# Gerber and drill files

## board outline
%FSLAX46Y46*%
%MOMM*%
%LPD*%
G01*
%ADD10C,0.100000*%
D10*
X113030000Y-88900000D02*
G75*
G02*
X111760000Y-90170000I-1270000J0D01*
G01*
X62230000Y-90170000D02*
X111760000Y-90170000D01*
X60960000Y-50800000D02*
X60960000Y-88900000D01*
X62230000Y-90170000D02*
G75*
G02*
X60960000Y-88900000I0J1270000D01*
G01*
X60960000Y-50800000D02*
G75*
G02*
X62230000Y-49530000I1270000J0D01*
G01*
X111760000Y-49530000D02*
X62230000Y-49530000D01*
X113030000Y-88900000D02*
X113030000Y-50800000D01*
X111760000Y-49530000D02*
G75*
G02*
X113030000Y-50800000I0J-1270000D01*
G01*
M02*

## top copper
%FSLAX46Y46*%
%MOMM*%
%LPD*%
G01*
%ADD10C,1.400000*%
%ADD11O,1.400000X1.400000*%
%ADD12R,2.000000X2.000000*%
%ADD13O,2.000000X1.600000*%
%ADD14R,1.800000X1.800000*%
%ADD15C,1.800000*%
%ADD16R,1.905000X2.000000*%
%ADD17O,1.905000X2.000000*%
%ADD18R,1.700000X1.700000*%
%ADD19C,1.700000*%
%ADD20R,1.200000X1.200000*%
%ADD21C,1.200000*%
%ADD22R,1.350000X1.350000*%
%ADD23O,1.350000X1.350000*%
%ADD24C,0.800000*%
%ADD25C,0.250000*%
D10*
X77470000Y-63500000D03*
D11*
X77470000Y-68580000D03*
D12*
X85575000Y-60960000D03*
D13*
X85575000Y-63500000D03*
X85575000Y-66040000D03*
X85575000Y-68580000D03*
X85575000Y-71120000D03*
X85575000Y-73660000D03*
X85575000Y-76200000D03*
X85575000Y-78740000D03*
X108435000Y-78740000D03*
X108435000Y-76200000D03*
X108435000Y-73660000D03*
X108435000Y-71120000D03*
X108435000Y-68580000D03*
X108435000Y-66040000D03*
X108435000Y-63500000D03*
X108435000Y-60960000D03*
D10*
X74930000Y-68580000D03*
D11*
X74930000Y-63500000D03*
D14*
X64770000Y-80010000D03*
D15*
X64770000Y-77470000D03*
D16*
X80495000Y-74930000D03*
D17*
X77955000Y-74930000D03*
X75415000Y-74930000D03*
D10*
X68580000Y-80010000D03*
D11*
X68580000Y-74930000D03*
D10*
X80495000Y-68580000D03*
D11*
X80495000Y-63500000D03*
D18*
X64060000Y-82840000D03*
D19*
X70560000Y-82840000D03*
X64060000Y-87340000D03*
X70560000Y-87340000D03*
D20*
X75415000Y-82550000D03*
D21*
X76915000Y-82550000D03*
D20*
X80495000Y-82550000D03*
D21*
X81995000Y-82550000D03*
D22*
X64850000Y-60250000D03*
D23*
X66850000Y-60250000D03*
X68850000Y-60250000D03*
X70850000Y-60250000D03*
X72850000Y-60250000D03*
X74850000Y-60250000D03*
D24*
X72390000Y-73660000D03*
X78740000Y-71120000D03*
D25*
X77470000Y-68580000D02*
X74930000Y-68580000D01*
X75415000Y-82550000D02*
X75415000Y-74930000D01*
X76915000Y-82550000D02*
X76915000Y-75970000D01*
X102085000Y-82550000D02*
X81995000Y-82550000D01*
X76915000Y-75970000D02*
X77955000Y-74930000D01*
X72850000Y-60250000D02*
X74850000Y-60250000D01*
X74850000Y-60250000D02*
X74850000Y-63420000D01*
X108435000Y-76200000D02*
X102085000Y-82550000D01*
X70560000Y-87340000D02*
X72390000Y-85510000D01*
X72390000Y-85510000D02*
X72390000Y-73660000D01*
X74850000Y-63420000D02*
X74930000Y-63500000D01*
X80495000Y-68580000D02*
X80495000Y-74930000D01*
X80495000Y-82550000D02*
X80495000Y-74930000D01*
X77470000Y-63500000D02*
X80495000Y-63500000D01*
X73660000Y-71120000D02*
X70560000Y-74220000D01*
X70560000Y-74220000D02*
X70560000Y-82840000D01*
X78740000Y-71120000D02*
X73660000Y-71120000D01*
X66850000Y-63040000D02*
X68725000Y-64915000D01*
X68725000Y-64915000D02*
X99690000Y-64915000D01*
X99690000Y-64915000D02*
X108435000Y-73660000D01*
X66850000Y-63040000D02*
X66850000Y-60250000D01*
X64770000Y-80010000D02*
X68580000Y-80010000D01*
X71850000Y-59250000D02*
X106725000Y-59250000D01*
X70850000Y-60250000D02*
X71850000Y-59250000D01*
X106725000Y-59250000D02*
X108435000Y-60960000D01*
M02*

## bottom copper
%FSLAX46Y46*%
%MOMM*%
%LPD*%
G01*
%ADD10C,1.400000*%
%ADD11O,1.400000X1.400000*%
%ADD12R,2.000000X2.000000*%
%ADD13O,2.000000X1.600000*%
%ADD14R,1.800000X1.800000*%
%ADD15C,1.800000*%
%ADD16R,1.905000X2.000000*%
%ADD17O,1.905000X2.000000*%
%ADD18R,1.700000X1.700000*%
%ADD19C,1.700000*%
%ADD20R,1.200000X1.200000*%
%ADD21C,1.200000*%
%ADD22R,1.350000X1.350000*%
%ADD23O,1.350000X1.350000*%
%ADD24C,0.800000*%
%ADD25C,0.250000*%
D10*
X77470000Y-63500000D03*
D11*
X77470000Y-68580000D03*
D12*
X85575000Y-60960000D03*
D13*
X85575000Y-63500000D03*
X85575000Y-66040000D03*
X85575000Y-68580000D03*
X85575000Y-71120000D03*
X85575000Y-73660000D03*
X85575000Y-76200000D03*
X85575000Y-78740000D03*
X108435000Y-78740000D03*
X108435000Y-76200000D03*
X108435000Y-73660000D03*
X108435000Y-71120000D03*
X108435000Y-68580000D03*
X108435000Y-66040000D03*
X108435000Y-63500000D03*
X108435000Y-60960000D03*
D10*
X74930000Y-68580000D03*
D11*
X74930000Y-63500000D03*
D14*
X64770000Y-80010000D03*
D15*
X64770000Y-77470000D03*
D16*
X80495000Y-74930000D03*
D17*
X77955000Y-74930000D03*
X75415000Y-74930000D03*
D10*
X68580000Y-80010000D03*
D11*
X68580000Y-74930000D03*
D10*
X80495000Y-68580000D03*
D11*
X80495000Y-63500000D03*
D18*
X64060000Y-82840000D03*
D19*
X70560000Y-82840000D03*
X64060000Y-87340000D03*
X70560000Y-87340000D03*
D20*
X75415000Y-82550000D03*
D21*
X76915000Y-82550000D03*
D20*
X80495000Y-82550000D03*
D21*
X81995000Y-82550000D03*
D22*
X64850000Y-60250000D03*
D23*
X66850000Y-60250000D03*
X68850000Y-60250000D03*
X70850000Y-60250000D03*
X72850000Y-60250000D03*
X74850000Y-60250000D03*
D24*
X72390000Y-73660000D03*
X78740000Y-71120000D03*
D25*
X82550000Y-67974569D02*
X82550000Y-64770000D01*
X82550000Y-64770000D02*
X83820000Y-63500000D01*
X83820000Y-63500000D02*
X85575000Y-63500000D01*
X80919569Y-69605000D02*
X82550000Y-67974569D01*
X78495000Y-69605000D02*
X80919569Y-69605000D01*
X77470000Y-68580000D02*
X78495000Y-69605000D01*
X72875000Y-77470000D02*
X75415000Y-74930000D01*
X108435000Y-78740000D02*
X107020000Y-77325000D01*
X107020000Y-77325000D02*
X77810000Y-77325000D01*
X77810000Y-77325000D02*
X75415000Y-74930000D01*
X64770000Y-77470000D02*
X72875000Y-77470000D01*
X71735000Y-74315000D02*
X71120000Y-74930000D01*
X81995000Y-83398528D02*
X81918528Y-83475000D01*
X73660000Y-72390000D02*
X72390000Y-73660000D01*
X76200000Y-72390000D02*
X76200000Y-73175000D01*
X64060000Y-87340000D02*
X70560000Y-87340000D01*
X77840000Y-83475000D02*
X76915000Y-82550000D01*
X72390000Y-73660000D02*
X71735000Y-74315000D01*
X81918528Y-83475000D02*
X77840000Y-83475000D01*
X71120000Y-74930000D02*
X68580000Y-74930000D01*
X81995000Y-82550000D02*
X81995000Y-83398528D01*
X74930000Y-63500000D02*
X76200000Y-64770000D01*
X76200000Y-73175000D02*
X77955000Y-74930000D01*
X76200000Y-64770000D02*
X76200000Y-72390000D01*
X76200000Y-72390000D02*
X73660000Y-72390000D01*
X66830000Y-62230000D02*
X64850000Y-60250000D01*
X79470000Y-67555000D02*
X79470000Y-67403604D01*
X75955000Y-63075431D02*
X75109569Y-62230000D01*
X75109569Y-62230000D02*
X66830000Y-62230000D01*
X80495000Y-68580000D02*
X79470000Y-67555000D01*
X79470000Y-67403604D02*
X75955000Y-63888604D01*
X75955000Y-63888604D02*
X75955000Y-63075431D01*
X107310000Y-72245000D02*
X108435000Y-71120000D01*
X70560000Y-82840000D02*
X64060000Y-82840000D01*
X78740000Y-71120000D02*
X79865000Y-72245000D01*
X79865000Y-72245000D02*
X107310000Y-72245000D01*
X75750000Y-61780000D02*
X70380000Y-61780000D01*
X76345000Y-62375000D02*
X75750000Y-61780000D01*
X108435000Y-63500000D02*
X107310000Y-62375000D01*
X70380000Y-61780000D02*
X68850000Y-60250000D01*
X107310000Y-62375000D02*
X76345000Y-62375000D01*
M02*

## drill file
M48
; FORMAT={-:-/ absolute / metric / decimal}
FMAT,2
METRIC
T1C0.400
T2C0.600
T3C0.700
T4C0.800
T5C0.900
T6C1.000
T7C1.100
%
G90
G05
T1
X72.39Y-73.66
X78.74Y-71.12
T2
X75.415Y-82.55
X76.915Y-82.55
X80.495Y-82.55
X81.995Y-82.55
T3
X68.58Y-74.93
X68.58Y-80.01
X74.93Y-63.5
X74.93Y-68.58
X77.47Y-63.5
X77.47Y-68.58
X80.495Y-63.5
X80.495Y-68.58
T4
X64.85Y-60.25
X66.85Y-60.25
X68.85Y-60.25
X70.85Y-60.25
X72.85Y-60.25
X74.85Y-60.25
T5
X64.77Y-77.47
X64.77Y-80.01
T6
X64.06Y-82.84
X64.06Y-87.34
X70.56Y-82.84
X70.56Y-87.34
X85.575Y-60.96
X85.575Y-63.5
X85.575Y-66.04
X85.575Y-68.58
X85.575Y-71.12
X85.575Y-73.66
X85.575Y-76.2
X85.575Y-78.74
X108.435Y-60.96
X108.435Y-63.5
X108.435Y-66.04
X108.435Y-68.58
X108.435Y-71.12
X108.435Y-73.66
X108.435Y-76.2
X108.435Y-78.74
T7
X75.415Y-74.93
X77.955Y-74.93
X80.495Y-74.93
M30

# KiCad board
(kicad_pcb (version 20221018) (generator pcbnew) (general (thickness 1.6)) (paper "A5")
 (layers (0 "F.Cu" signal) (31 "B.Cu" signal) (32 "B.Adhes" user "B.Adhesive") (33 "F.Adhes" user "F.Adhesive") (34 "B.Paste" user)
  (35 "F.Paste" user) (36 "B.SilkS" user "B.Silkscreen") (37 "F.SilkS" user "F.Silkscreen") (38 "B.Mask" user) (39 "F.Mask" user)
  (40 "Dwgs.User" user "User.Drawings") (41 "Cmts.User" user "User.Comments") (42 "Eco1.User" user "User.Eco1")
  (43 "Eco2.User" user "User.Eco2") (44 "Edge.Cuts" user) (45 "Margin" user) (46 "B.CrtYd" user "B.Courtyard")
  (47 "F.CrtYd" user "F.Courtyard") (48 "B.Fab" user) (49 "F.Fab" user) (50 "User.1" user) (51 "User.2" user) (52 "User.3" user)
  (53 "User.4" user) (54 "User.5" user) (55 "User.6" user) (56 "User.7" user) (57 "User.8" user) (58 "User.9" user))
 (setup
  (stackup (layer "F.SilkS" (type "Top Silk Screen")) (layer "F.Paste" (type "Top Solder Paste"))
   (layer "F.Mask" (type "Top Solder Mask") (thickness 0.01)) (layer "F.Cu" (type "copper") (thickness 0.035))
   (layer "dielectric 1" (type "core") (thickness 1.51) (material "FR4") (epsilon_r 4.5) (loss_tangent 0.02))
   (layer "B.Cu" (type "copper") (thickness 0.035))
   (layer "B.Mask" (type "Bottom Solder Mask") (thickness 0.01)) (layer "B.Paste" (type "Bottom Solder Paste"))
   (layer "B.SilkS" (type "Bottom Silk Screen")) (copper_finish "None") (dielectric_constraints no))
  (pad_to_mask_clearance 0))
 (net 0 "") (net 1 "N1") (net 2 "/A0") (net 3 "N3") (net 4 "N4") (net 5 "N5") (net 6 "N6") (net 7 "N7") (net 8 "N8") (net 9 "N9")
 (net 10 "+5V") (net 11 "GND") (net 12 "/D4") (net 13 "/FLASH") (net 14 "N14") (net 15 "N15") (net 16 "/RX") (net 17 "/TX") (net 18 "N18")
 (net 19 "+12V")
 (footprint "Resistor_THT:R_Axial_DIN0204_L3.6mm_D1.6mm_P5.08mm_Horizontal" (layer "F.Cu") (at 77.47 63.5 -90)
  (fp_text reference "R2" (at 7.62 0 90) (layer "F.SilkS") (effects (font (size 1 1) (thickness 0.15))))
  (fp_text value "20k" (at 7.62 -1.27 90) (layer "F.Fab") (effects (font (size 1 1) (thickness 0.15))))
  (pad "1" thru_hole circle (at 0 0 270) (size 1.4 1.4) (drill 0.7) (layers "*.Cu" "*.Mask") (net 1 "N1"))
  (pad "2" thru_hole oval (at 5.08 0 270) (size 1.4 1.4) (drill 0.7) (layers "*.Cu" "*.Mask") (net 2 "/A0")))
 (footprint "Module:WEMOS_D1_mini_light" (layer "F.Cu") (at 85.575 60.96)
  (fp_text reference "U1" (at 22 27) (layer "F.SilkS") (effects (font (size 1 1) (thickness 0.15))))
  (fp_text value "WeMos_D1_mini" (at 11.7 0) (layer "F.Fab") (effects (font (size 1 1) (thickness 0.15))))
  (pad "1" thru_hole rect (at 0 0) (size 2 2) (drill 1) (layers "*.Cu" "*.Mask") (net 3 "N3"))
  (pad "2" thru_hole oval (at 0 2.54) (size 2 1.6) (drill 1) (layers "*.Cu" "*.Mask") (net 2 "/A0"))
  (pad "3" thru_hole oval (at 0 5.08) (size 2 1.6) (drill 1) (layers "*.Cu" "*.Mask") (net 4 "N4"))
  (pad "4" thru_hole oval (at 0 7.62) (size 2 1.6) (drill 1) (layers "*.Cu" "*.Mask") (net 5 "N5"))
  (pad "5" thru_hole oval (at 0 10.16) (size 2 1.6) (drill 1) (layers "*.Cu" "*.Mask") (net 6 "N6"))
  (pad "6" thru_hole oval (at 0 12.7) (size 2 1.6) (drill 1) (layers "*.Cu" "*.Mask") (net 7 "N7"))
  (pad "7" thru_hole oval (at 0 15.24) (size 2 1.6) (drill 1) (layers "*.Cu" "*.Mask") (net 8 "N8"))
  (pad "8" thru_hole oval (at 0 17.78) (size 2 1.6) (drill 1) (layers "*.Cu" "*.Mask") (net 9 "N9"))
  (pad "9" thru_hole oval (at 22.86 17.78) (size 2 1.6) (drill 1) (layers "*.Cu" "*.Mask") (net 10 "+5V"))
  (pad "10" thru_hole oval (at 22.86 15.24) (size 2 1.6) (drill 1) (layers "*.Cu" "*.Mask") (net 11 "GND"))
  (pad "11" thru_hole oval (at 22.86 12.7) (size 2 1.6) (drill 1) (layers "*.Cu" "*.Mask") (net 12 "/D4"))
  (pad "12" thru_hole oval (at 22.86 10.16) (size 2 1.6) (drill 1) (layers "*.Cu" "*.Mask") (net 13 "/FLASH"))
  (pad "13" thru_hole oval (at 22.86 7.62) (size 2 1.6) (drill 1) (layers "*.Cu" "*.Mask") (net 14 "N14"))
  (pad "14" thru_hole oval (at 22.86 5.08) (size 2 1.6) (drill 1) (layers "*.Cu" "*.Mask") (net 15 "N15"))
  (pad "15" thru_hole oval (at 22.86 2.54) (size 2 1.6) (drill 1) (layers "*.Cu" "*.Mask") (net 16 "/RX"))
  (pad "16" thru_hole oval (at 22.86 0) (size 2 1.6) (drill 1) (layers "*.Cu" "*.Mask") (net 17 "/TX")))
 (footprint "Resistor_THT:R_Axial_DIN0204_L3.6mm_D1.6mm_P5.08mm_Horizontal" (layer "F.Cu") (at 74.93 68.58 90)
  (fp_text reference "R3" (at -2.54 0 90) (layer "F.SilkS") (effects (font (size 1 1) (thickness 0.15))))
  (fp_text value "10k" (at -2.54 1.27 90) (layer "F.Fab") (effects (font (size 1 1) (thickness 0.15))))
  (pad "1" thru_hole circle (at 0 0 90) (size 1.4 1.4) (drill 0.7) (layers "*.Cu" "*.Mask") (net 2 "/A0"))
  (pad "2" thru_hole oval (at 5.08 0 90) (size 1.4 1.4) (drill 0.7) (layers "*.Cu" "*.Mask") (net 11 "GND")))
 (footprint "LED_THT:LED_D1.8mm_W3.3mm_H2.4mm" (layer "F.Cu") (at 64.77 80.01 90)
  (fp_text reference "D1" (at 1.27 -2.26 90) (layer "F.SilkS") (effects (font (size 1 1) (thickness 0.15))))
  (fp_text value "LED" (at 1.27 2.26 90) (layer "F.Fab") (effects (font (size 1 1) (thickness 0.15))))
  (pad "1" thru_hole rect (at 0 0 90) (size 1.8 1.8) (drill 0.9) (layers "*.Cu" "*.Mask") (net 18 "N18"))
  (pad "2" thru_hole circle (at 2.54 0 90) (size 1.8 1.8) (drill 0.9) (layers "*.Cu" "*.Mask") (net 10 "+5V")))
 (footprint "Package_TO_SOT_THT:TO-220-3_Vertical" (layer "F.Cu") (at 80.495 74.93 180)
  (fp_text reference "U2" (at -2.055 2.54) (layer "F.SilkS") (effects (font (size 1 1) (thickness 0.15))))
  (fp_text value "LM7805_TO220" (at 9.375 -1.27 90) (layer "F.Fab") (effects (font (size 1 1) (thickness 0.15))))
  (pad "1" thru_hole rect (at 0 0 180) (size 1.905 2) (drill 1.1) (layers "*.Cu" "*.Mask") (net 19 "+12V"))
  (pad "2" thru_hole oval (at 2.54 0 180) (size 1.905 2) (drill 1.1) (layers "*.Cu" "*.Mask") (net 11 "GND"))
  (pad "3" thru_hole oval (at 5.08 0 180) (size 1.905 2) (drill 1.1) (layers "*.Cu" "*.Mask") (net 10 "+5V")))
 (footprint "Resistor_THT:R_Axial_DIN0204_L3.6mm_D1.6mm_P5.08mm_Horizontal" (layer "F.Cu") (at 68.58 80.01 90)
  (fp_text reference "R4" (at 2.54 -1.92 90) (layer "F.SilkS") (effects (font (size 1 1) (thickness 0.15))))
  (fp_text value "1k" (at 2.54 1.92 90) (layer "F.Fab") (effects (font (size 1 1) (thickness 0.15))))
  (pad "1" thru_hole circle (at 0 0 90) (size 1.4 1.4) (drill 0.7) (layers "*.Cu" "*.Mask") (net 18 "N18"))
  (pad "2" thru_hole oval (at 5.08 0 90) (size 1.4 1.4) (drill 0.7) (layers "*.Cu" "*.Mask") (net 11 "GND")))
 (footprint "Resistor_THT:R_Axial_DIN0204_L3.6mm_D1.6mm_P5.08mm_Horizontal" (layer "F.Cu") (at 80.495 68.58 90)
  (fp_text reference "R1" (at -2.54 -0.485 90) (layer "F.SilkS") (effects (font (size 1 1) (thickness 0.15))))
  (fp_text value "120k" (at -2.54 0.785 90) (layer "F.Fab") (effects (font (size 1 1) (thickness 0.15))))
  (pad "1" thru_hole circle (at 0 0 90) (size 1.4 1.4) (drill 0.7) (layers "*.Cu" "*.Mask") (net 19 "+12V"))
  (pad "2" thru_hole oval (at 5.08 0 90) (size 1.4 1.4) (drill 0.7) (layers "*.Cu" "*.Mask") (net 1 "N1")))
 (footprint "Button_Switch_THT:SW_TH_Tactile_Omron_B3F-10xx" (layer "F.Cu") (at 64.06 82.84)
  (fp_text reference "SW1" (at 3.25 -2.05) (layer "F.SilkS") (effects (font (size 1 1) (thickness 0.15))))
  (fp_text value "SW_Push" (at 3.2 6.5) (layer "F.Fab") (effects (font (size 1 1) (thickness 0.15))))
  (pad "1" thru_hole rect (at 0 0) (size 1.7 1.7) (drill 1) (layers "*.Cu" "*.Mask") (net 13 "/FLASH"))
  (pad "1" thru_hole circle (at 6.5 0) (size 1.7 1.7) (drill 1) (layers "*.Cu" "*.Mask") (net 13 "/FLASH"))
  (pad "2" thru_hole circle (at 0 4.5) (size 1.7 1.7) (drill 1) (layers "*.Cu" "*.Mask") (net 11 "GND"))
  (pad "2" thru_hole circle (at 6.5 4.5) (size 1.7 1.7) (drill 1) (layers "*.Cu" "*.Mask") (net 11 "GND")))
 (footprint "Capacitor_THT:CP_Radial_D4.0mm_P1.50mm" (layer "F.Cu") (at 75.415 82.55)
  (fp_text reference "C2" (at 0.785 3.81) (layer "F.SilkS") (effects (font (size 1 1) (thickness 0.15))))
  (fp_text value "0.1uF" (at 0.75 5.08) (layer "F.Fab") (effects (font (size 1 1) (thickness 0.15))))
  (pad "1" thru_hole rect (at 0 0) (size 1.2 1.2) (drill 0.6) (layers "*.Cu" "*.Mask") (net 10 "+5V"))
  (pad "2" thru_hole circle (at 1.5 0) (size 1.2 1.2) (drill 0.6) (layers "*.Cu" "*.Mask") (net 11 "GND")))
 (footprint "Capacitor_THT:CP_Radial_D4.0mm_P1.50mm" (layer "F.Cu") (at 80.495 82.55)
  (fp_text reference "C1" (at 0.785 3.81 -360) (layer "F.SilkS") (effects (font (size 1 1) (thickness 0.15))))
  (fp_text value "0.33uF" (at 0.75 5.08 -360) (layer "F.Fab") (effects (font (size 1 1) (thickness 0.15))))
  (pad "1" thru_hole rect (at 0 0) (size 1.2 1.2) (drill 0.6) (layers "*.Cu" "*.Mask") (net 19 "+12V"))
  (pad "2" thru_hole circle (at 1.5 0) (size 1.2 1.2) (drill 0.6) (layers "*.Cu" "*.Mask") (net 11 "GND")))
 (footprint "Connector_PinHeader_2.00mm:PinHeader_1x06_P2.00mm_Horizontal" (layer "F.Cu") (at 64.85 60.25 90)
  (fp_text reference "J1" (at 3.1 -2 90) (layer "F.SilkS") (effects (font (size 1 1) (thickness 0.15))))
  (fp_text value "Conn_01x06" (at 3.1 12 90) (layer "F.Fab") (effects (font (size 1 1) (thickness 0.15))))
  (pad "1" thru_hole rect (at 0 0 90) (size 1.35 1.35) (drill 0.8) (layers "*.Cu" "*.Mask") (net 19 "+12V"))
  (pad "2" thru_hole oval (at 0 2 90) (size 1.35 1.35) (drill 0.8) (layers "*.Cu" "*.Mask") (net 12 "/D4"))
  (pad "3" thru_hole oval (at 0 4 90) (size 1.35 1.35) (drill 0.8) (layers "*.Cu" "*.Mask") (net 16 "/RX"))
  (pad "4" thru_hole oval (at 0 6 90) (size 1.35 1.35) (drill 0.8) (layers "*.Cu" "*.Mask") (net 17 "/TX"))
  (pad "5" thru_hole oval (at 0 8 90) (size 1.35 1.35) (drill 0.8) (layers "*.Cu" "*.Mask") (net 11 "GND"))
  (pad "6" thru_hole oval (at 0 10 90) (size 1.35 1.35) (drill 0.8) (layers "*.Cu" "*.Mask") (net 11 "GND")))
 (gr_arc locked (start 113.03 88.9) (mid 112.658026 89.798026) (end 111.76 90.17) (stroke (width 0.1) (type default)) (layer "Edge.Cuts"))
 (gr_line locked (start 62.23 90.17) (end 111.76 90.17) (stroke (width 0.1) (type default)) (layer "Edge.Cuts"))
 (gr_line locked (start 60.96 50.8) (end 60.96 88.9) (stroke (width 0.1) (type default)) (layer "Edge.Cuts"))
 (gr_arc locked (start 62.23 90.17) (mid 61.331974 89.798026) (end 60.96 88.9) (stroke (width 0.1) (type default)) (layer "Edge.Cuts"))
 (gr_arc locked (start 60.96 50.8) (mid 61.331974 49.901974) (end 62.23 49.53) (stroke (width 0.1) (type default)) (layer "Edge.Cuts"))
 (gr_line locked (start 111.76 49.53) (end 62.23 49.53) (stroke (width 0.1) (type default)) (layer "Edge.Cuts"))
 (gr_line locked (start 113.03 88.9) (end 113.03 50.8) (stroke (width 0.1) (type default)) (layer "Edge.Cuts"))
 (gr_arc locked (start 111.76 49.53) (mid 112.658026 49.901974) (end 113.03 50.8) (stroke (width 0.1) (type default)) (layer "Edge.Cuts"))
 (segment (start 77.47 68.58) (end 74.93 68.58) (width 0.25) (layer "F.Cu") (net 2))
 (segment (start 82.55 67.974569) (end 82.55 64.77) (width 0.25) (layer "B.Cu") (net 2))
 (segment (start 82.55 64.77) (end 83.82 63.5) (width 0.25) (layer "B.Cu") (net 2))
 (segment (start 83.82 63.5) (end 85.575 63.5) (width 0.25) (layer "B.Cu") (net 2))
 (segment (start 80.919569 69.605) (end 82.55 67.974569) (width 0.25) (layer "B.Cu") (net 2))
 (segment (start 78.495 69.605) (end 80.919569 69.605) (width 0.25) (layer "B.Cu") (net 2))
 (segment (start 77.47 68.58) (end 78.495 69.605) (width 0.25) (layer "B.Cu") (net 2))
 (segment (start 75.415 82.55) (end 75.415 74.93) (width 0.25) (layer "F.Cu") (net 10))
 (segment (start 72.875 77.47) (end 75.415 74.93) (width 0.25) (layer "B.Cu") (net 10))
 (segment (start 108.435 78.74) (end 107.02 77.325) (width 0.25) (layer "B.Cu") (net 10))
 (segment (start 107.02 77.325) (end 77.81 77.325) (width 0.25) (layer "B.Cu") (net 10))
 (segment (start 77.81 77.325) (end 75.415 74.93) (width 0.25) (layer "B.Cu") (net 10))
 (segment (start 64.77 77.47) (end 72.875 77.47) (width 0.25) (layer "B.Cu") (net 10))
 (segment (start 76.915 82.55) (end 76.915 75.97) (width 0.25) (layer "F.Cu") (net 11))
 (segment (start 102.085 82.55) (end 81.995 82.55) (width 0.25) (layer "F.Cu") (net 11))
 (segment (start 76.915 75.97) (end 77.955 74.93) (width 0.25) (layer "F.Cu") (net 11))
 (segment (start 72.85 60.25) (end 74.85 60.25) (width 0.25) (layer "F.Cu") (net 11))
 (segment (start 74.85 60.25) (end 74.85 63.42) (width 0.25) (layer "F.Cu") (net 11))
 (segment (start 108.435 76.2) (end 102.085 82.55) (width 0.25) (layer "F.Cu") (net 11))
 (segment (start 70.56 87.34) (end 72.39 85.51) (width 0.25) (layer "F.Cu") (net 11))
 (segment (start 72.39 85.51) (end 72.39 73.66) (width 0.25) (layer "F.Cu") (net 11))
 (segment (start 74.85 63.42) (end 74.93 63.5) (width 0.25) (layer "F.Cu") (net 11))
 (via (at 72.39 73.66) (size 0.8) (drill 0.4) (layers "F.Cu" "B.Cu") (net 11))
 (segment (start 71.735 74.315) (end 71.12 74.93) (width 0.25) (layer "B.Cu") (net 11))
 (segment (start 81.995 83.398528) (end 81.918528 83.475) (width 0.25) (layer "B.Cu") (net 11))
 (segment (start 73.66 72.39) (end 72.39 73.66) (width 0.25) (layer "B.Cu") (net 11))
 (segment (start 76.2 72.39) (end 76.2 73.175) (width 0.25) (layer "B.Cu") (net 11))
 (segment (start 64.06 87.34) (end 70.56 87.34) (width 0.25) (layer "B.Cu") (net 11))
 (segment (start 77.84 83.475) (end 76.915 82.55) (width 0.25) (layer "B.Cu") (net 11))
 (segment (start 72.39 73.66) (end 71.735 74.315) (width 0.25) (layer "B.Cu") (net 11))
 (segment (start 81.918528 83.475) (end 77.84 83.475) (width 0.25) (layer "B.Cu") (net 11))
 (segment (start 71.12 74.93) (end 68.58 74.93) (width 0.25) (layer "B.Cu") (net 11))
 (segment (start 81.995 82.55) (end 81.995 83.398528) (width 0.25) (layer "B.Cu") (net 11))
 (segment (start 74.93 63.5) (end 76.2 64.77) (width 0.25) (layer "B.Cu") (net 11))
 (segment (start 76.2 73.175) (end 77.955 74.93) (width 0.25) (layer "B.Cu") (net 11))
 (segment (start 76.2 64.77) (end 76.2 72.39) (width 0.25) (layer "B.Cu") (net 11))
 (segment (start 76.2 72.39) (end 73.66 72.39) (width 0.25) (layer "B.Cu") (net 11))
 (segment (start 80.495 68.58) (end 80.495 74.93) (width 0.25) (layer "F.Cu") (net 19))
 (segment (start 80.495 82.55) (end 80.495 74.93) (width 0.25) (layer "F.Cu") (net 19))
 (segment (start 66.83 62.23) (end 64.85 60.25) (width 0.25) (layer "B.Cu") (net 19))
 (segment (start 79.47 67.555) (end 79.47 67.403604) (width 0.25) (layer "B.Cu") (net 19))
 (segment (start 75.955 63.075431) (end 75.109569 62.23) (width 0.25) (layer "B.Cu") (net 19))
 (segment (start 75.109569 62.23) (end 66.83 62.23) (width 0.25) (layer "B.Cu") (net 19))
 (segment (start 80.495 68.58) (end 79.47 67.555) (width 0.25) (layer "B.Cu") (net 19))
 (segment (start 79.47 67.403604) (end 75.955 63.888604) (width 0.25) (layer "B.Cu") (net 19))
 (segment (start 75.955 63.888604) (end 75.955 63.075431) (width 0.25) (layer "B.Cu") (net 19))
 (segment (start 77.47 63.5) (end 80.495 63.5) (width 0.25) (layer "F.Cu") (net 1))
 (segment (start 73.66 71.12) (end 70.56 74.22) (width 0.25) (layer "F.Cu") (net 13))
 (segment (start 70.56 74.22) (end 70.56 82.84) (width 0.25) (layer "F.Cu") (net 13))
 (segment (start 78.74 71.12) (end 73.66 71.12) (width 0.25) (layer "F.Cu") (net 13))
 (via (at 78.74 71.12) (size 0.8) (drill 0.4) (layers "F.Cu" "B.Cu") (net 13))
 (segment (start 107.31 72.245) (end 108.435 71.12) (width 0.25) (layer "B.Cu") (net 13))
 (segment (start 70.56 82.84) (end 64.06 82.84) (width 0.25) (layer "B.Cu") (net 13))
 (segment (start 78.74 71.12) (end 79.865 72.245) (width 0.25) (layer "B.Cu") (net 13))
 (segment (start 79.865 72.245) (end 107.31 72.245) (width 0.25) (layer "B.Cu") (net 13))
 (segment (start 66.85 63.04) (end 68.725 64.915) (width 0.25) (layer "F.Cu") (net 12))
 (segment (start 68.725 64.915) (end 99.69 64.915) (width 0.25) (layer "F.Cu") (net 12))
 (segment (start 99.69 64.915) (end 108.435 73.66) (width 0.25) (layer "F.Cu") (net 12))
 (segment (start 66.85 63.04) (end 66.85 60.25) (width 0.25) (layer "F.Cu") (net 12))
 (segment (start 64.77 80.01) (end 68.58 80.01) (width 0.25) (layer "F.Cu") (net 18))
 (segment (start 75.75 61.78) (end 70.38 61.78) (width 0.25) (layer "B.Cu") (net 16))
 (segment (start 76.345 62.375) (end 75.75 61.78) (width 0.25) (layer "B.Cu") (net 16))
 (segment (start 108.435 63.5) (end 107.31 62.375) (width 0.25) (layer "B.Cu") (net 16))
 (segment (start 70.38 61.78) (end 68.85 60.25) (width 0.25) (layer "B.Cu") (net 16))
 (segment (start 107.31 62.375) (end 76.345 62.375) (width 0.25) (layer "B.Cu") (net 16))
 (segment (start 71.85 59.25) (end 106.725 59.25) (width 0.25) (layer "F.Cu") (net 17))
 (segment (start 70.85 60.25) (end 71.85 59.25) (width 0.25) (layer "F.Cu") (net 17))
 (segment (start 106.725 59.25) (end 108.435 60.96) (width 0.25) (layer "F.Cu") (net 17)))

